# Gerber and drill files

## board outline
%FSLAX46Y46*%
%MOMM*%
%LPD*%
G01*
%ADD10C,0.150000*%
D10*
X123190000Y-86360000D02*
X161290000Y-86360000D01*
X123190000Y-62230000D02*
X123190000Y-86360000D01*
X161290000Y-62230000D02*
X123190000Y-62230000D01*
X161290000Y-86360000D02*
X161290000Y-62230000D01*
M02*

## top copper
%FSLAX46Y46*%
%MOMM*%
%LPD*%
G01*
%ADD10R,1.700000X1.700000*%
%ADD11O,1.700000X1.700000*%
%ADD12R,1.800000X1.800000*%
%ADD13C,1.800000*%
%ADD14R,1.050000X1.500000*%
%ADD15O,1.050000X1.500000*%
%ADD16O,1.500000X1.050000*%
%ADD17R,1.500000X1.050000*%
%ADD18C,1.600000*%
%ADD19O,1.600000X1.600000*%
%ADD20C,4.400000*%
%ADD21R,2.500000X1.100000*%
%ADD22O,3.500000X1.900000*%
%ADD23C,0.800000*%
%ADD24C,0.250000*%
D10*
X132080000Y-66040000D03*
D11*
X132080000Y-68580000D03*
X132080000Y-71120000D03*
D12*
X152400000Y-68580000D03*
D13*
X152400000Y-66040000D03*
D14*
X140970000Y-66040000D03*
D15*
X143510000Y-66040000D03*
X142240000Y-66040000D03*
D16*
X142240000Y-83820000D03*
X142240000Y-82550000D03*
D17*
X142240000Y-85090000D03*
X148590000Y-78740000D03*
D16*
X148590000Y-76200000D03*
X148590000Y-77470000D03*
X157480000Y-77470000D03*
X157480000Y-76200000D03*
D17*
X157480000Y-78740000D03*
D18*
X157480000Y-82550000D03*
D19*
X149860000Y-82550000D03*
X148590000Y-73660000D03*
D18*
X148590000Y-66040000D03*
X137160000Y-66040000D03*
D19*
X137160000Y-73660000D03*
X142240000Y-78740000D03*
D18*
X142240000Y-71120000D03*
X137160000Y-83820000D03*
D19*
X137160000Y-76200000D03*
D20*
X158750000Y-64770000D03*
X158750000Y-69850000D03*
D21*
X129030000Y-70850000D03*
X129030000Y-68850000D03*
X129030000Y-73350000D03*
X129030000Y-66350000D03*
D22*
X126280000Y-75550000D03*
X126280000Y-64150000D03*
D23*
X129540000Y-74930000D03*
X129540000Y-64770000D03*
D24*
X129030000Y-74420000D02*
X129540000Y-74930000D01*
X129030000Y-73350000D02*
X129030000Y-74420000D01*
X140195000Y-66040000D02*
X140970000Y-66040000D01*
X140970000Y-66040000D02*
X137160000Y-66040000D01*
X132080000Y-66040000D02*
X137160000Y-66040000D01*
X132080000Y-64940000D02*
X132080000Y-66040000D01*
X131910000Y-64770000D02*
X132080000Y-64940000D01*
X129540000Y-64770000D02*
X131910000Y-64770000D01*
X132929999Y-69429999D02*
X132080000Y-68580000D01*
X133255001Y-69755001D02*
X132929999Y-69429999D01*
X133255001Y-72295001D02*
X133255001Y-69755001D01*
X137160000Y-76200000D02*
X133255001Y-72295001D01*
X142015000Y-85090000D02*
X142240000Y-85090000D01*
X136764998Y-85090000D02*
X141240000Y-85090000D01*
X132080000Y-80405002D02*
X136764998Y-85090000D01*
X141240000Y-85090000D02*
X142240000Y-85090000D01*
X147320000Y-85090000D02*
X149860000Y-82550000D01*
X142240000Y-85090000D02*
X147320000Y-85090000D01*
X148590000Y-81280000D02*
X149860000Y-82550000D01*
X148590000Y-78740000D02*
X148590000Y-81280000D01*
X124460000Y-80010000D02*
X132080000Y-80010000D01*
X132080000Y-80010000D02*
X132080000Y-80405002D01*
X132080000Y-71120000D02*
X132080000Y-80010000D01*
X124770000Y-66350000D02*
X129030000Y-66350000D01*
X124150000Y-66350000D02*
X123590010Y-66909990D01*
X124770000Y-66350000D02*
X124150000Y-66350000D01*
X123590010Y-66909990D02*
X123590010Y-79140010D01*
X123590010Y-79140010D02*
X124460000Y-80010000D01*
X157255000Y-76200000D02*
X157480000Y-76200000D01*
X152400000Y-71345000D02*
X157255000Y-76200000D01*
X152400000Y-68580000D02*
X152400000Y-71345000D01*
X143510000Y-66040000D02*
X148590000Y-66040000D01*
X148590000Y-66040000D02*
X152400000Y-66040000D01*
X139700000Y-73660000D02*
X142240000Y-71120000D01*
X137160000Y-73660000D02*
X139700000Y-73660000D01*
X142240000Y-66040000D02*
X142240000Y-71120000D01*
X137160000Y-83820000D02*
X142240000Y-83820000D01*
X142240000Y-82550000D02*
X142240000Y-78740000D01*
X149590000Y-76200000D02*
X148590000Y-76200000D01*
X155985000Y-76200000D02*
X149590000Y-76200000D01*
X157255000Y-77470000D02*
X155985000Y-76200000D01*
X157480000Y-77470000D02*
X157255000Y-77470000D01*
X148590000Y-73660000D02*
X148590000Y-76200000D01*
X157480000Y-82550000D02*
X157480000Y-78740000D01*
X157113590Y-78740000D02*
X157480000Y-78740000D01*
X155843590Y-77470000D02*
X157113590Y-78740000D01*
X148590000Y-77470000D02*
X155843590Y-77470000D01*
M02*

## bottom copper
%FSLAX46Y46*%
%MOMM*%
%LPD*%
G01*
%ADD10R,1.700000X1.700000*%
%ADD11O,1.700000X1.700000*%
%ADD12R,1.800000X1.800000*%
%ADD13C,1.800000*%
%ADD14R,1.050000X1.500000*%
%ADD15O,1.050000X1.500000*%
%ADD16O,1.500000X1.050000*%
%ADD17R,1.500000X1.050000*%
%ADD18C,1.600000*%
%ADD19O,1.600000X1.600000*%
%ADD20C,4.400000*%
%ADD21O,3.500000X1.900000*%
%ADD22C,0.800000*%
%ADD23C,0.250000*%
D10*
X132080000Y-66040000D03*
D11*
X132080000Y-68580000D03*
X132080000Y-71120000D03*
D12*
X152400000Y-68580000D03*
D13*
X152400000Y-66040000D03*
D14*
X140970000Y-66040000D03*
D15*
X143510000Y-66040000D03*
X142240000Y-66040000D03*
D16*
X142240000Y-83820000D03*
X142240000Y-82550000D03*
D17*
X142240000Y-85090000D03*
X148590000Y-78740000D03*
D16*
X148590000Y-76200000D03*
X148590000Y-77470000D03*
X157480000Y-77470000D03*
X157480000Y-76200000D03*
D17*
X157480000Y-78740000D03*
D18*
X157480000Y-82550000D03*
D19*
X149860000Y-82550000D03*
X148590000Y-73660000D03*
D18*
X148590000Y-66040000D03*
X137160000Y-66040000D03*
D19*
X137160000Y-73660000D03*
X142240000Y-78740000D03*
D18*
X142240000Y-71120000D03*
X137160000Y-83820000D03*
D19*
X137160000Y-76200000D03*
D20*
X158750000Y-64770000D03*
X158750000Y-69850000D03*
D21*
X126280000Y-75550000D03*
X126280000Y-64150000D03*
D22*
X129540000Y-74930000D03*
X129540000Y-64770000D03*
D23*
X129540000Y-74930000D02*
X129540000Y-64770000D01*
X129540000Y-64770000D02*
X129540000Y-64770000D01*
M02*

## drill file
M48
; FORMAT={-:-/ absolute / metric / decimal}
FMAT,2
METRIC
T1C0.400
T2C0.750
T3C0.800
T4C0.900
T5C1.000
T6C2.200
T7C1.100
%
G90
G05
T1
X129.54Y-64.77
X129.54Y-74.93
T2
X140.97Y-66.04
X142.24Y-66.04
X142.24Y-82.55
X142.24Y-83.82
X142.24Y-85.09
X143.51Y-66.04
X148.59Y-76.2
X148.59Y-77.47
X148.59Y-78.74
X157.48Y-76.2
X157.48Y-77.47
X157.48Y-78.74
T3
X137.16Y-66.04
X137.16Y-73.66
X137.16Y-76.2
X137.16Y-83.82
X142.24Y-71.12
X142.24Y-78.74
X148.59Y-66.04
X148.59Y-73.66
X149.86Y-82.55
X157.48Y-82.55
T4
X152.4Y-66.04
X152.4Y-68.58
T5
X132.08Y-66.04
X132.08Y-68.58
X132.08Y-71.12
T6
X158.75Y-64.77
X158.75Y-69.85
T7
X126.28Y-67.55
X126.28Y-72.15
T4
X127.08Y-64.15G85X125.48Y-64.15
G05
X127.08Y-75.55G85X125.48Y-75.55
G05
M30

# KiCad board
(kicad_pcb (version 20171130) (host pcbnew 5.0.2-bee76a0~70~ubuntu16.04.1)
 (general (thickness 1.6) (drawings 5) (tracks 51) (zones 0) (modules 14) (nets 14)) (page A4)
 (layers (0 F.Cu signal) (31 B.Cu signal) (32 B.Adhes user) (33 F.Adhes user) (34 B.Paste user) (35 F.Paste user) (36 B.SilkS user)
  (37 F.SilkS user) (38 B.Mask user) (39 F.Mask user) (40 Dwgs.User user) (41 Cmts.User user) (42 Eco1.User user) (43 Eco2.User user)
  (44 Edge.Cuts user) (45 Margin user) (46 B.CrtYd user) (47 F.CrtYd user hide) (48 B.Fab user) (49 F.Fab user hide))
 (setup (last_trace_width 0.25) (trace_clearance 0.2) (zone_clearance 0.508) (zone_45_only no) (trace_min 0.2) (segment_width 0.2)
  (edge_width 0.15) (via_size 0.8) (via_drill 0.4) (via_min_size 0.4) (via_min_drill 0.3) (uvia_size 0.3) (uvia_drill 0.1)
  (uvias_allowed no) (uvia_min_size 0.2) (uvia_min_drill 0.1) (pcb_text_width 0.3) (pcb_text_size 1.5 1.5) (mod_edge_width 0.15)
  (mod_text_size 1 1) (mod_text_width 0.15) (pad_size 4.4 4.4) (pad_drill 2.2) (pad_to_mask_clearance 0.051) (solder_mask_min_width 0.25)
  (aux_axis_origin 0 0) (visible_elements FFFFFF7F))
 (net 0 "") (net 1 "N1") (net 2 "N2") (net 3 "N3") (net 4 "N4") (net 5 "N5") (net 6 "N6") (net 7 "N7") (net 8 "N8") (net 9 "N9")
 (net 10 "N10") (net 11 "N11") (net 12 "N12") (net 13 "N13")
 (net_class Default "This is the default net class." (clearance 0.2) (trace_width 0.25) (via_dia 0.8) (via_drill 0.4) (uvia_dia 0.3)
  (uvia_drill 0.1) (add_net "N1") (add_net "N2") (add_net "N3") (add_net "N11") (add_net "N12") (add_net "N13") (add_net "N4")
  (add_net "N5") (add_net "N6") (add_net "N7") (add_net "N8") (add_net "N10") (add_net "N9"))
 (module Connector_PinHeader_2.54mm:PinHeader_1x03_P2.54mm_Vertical (layer F.Cu) (at 132.08 66.04)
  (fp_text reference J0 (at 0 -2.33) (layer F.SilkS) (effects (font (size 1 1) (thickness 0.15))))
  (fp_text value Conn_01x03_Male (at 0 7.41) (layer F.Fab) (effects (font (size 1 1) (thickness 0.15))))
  (pad 1 thru_hole rect (at 0 0) (size 1.7 1.7) (drill 1) (layers *.Cu *.Mask) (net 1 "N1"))
  (pad 2 thru_hole oval (at 0 2.54) (size 1.7 1.7) (drill 1) (layers *.Cu *.Mask) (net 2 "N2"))
  (pad 3 thru_hole oval (at 0 5.08) (size 1.7 1.7) (drill 1) (layers *.Cu *.Mask) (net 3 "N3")))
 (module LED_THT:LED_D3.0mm (layer F.Cu) (at 152.4 68.58 90)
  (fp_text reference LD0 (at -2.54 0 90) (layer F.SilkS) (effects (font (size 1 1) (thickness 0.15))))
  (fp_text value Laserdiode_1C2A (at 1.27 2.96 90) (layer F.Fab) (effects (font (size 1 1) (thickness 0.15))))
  (pad 1 thru_hole rect (at 0 0 90) (size 1.8 1.8) (drill 0.9) (layers *.Cu *.Mask) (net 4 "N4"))
  (pad 2 thru_hole circle (at 2.54 0 90) (size 1.8 1.8) (drill 0.9) (layers *.Cu *.Mask) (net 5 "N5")))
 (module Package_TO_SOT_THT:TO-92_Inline (layer F.Cu) (at 140.97 66.04)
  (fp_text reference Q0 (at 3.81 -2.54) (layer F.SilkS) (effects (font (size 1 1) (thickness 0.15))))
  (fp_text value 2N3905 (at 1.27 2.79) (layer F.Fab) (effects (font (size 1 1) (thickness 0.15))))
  (pad 1 thru_hole rect (at 0 0) (size 1.05 1.5) (drill 0.75) (layers *.Cu *.Mask) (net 1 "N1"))
  (pad 3 thru_hole oval (at 2.54 0) (size 1.05 1.5) (drill 0.75) (layers *.Cu *.Mask) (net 5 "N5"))
  (pad 2 thru_hole oval (at 1.27 0) (size 1.05 1.5) (drill 0.75) (layers *.Cu *.Mask) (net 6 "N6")))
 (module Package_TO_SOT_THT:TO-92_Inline (layer F.Cu) (at 142.24 85.09 90)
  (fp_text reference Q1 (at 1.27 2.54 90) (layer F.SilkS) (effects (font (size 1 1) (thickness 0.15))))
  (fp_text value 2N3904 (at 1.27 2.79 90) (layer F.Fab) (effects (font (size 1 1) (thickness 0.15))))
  (pad 2 thru_hole oval (at 1.27 0 90) (size 1.05 1.5) (drill 0.75) (layers *.Cu *.Mask) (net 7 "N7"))
  (pad 3 thru_hole oval (at 2.54 0 90) (size 1.05 1.5) (drill 0.75) (layers *.Cu *.Mask) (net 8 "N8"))
  (pad 1 thru_hole rect (at 0 0 90) (size 1.05 1.5) (drill 0.75) (layers *.Cu *.Mask) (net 3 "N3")))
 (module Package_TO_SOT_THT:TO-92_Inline (layer F.Cu) (at 148.59 78.74 90)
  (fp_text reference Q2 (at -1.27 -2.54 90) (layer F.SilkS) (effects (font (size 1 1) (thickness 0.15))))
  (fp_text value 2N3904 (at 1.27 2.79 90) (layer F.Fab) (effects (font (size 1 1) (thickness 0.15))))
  (pad 1 thru_hole rect (at 0 0 90) (size 1.05 1.5) (drill 0.75) (layers *.Cu *.Mask) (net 3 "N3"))
  (pad 3 thru_hole oval (at 2.54 0 90) (size 1.05 1.5) (drill 0.75) (layers *.Cu *.Mask) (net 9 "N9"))
  (pad 2 thru_hole oval (at 1.27 0 90) (size 1.05 1.5) (drill 0.75) (layers *.Cu *.Mask) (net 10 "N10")))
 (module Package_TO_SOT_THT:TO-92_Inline (layer F.Cu) (at 157.48 78.74 90)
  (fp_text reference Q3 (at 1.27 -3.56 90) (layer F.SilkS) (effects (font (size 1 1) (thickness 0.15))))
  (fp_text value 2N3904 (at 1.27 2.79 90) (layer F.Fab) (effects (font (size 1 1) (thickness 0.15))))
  (pad 2 thru_hole oval (at 1.27 0 90) (size 1.05 1.5) (drill 0.75) (layers *.Cu *.Mask) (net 9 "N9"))
  (pad 3 thru_hole oval (at 2.54 0 90) (size 1.05 1.5) (drill 0.75) (layers *.Cu *.Mask) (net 4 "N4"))
  (pad 1 thru_hole rect (at 0 0 90) (size 1.05 1.5) (drill 0.75) (layers *.Cu *.Mask) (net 10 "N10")))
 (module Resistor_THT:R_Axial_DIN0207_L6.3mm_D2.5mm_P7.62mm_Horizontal (layer F.Cu) (at 157.48 82.55 180)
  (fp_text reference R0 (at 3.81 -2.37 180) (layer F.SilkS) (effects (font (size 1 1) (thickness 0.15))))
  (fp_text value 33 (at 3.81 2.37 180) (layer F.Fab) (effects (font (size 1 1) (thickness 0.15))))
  (pad 1 thru_hole circle (at 0 0 180) (size 1.6 1.6) (drill 0.8) (layers *.Cu *.Mask) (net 10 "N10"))
  (pad 2 thru_hole oval (at 7.62 0 180) (size 1.6 1.6) (drill 0.8) (layers *.Cu *.Mask) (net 3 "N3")))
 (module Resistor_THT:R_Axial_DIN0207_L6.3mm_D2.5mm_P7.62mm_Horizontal (layer F.Cu) (at 148.59 66.04 270)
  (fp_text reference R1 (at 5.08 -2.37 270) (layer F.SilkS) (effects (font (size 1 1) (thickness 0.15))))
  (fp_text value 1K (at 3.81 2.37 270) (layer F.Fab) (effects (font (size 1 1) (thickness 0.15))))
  (pad 2 thru_hole oval (at 7.62 0 270) (size 1.6 1.6) (drill 0.8) (layers *.Cu *.Mask) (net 9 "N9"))
  (pad 1 thru_hole circle (at 0 0 270) (size 1.6 1.6) (drill 0.8) (layers *.Cu *.Mask) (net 5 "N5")))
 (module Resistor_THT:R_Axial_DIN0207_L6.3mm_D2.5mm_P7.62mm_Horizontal (layer F.Cu) (at 137.16 66.04 270)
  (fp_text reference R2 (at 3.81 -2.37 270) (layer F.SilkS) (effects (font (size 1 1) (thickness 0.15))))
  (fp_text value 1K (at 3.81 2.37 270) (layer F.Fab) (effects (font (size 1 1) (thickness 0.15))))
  (pad 1 thru_hole circle (at 0 0 270) (size 1.6 1.6) (drill 0.8) (layers *.Cu *.Mask) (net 1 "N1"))
  (pad 2 thru_hole oval (at 7.62 0 270) (size 1.6 1.6) (drill 0.8) (layers *.Cu *.Mask) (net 6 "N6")))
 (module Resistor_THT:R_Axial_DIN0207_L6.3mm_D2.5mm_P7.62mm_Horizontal (layer F.Cu) (at 142.24 71.12 270)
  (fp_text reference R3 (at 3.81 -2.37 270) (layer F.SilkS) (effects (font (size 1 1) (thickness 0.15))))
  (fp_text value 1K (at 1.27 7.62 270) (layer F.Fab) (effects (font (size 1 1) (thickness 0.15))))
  (pad 2 thru_hole oval (at 7.62 0 270) (size 1.6 1.6) (drill 0.8) (layers *.Cu *.Mask) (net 8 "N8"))
  (pad 1 thru_hole circle (at 0 0 270) (size 1.6 1.6) (drill 0.8) (layers *.Cu *.Mask) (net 6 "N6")))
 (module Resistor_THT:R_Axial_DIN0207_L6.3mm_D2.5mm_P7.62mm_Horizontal (layer F.Cu) (at 137.16 83.82 90)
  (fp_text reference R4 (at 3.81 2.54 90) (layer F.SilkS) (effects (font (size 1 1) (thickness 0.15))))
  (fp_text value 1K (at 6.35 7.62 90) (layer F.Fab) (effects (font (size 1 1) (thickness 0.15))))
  (pad 1 thru_hole circle (at 0 0 90) (size 1.6 1.6) (drill 0.8) (layers *.Cu *.Mask) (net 7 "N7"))
  (pad 2 thru_hole oval (at 7.62 0 90) (size 1.6 1.6) (drill 0.8) (layers *.Cu *.Mask) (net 2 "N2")))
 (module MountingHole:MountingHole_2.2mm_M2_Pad (layer F.Cu) (at 158.75 64.77)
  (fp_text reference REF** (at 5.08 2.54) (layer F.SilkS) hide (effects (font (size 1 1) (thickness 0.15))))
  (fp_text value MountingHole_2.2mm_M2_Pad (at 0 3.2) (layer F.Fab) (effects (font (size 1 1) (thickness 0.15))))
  (pad "" thru_hole circle (at 0 0) (size 4.4 4.4) (drill 2.2) (layers *.Cu *.Mask)))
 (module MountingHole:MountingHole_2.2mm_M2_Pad (layer F.Cu) (at 158.75 69.85)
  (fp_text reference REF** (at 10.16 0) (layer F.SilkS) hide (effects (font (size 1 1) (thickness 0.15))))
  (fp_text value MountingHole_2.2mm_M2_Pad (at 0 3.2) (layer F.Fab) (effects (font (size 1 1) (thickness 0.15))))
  (pad "" thru_hole circle (at 0 0) (size 4.4 4.4) (drill 2.2) (layers *.Cu *.Mask)))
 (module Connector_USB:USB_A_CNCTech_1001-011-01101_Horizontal (layer F.Cu) (at 119.38 69.85 180)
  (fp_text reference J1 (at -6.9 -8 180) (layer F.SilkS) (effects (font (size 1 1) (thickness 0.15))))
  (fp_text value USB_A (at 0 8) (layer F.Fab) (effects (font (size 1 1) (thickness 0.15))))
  (pad 2 smd rect (at -9.65 -1 180) (size 2.5 1.1) (layers F.Cu F.Paste F.Mask) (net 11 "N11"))
  (pad 3 smd rect (at -9.65 1 180) (size 2.5 1.1) (layers F.Cu F.Paste F.Mask) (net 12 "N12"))
  (pad 1 smd rect (at -9.65 -3.5 180) (size 2.5 1.1) (layers F.Cu F.Paste F.Mask) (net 1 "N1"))
  (pad 4 smd rect (at -9.65 3.5 180) (size 2.5 1.1) (layers F.Cu F.Paste F.Mask) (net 3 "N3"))
  (pad 5 thru_hole oval (at -6.9 -5.7 180) (size 3.5 1.9) (drill oval 2.5 0.9) (layers *.Cu *.Mask) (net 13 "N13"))
  (pad 5 thru_hole oval (at -6.9 5.7 180) (size 3.5 1.9) (drill oval 2.5 0.9) (layers *.Cu *.Mask) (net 13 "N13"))
  (pad "" np_thru_hole circle (at -6.9 -2.3 180) (size 1.1 1.1) (drill 1.1) (layers *.Cu *.Mask))
  (pad "" np_thru_hole circle (at -6.9 2.3 180) (size 1.1 1.1) (drill 1.1) (layers *.Cu *.Mask)))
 (gr_line (start 123.19 86.36) (end 161.29 86.36) (layer Edge.Cuts) (width 0.15))
 (gr_line (start 123.19 62.23) (end 123.19 86.36) (layer Edge.Cuts) (width 0.15))
 (gr_line (start 161.29 62.23) (end 123.19 62.23) (layer Edge.Cuts) (width 0.15))
 (gr_line (start 161.29 86.36) (end 161.29 62.23) (layer Edge.Cuts) (width 0.15))
 (via (at 129.54 74.93) (size 0.8) (drill 0.4) (layers F.Cu B.Cu) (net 1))
 (segment (start 129.03 74.42) (end 129.54 74.93) (width 0.25) (layer F.Cu) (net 1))
 (segment (start 129.03 73.35) (end 129.03 74.42) (width 0.25) (layer F.Cu) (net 1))
 (segment (start 129.54 74.93) (end 129.54 64.77) (width 0.25) (layer B.Cu) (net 1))
 (segment (start 129.54 64.77) (end 129.54 64.77) (width 0.25) (layer B.Cu) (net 1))
 (via (at 129.54 64.77) (size 0.8) (drill 0.4) (layers F.Cu B.Cu) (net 1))
 (segment (start 140.195 66.04) (end 140.97 66.04) (width 0.25) (layer F.Cu) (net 1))
 (segment (start 140.97 66.04) (end 137.16 66.04) (width 0.25) (layer F.Cu) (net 1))
 (segment (start 132.08 66.04) (end 137.16 66.04) (width 0.25) (layer F.Cu) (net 1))
 (segment (start 132.08 64.94) (end 132.08 66.04) (width 0.25) (layer F.Cu) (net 1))
 (segment (start 131.91 64.77) (end 132.08 64.94) (width 0.25) (layer F.Cu) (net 1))
 (segment (start 129.54 64.77) (end 131.91 64.77) (width 0.25) (layer F.Cu) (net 1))
 (segment (start 132.929999 69.429999) (end 132.08 68.58) (width 0.25) (layer F.Cu) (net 2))
 (segment (start 133.255001 69.755001) (end 132.929999 69.429999) (width 0.25) (layer F.Cu) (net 2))
 (segment (start 133.255001 72.295001) (end 133.255001 69.755001) (width 0.25) (layer F.Cu) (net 2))
 (segment (start 137.16 76.2) (end 133.255001 72.295001) (width 0.25) (layer F.Cu) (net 2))
 (segment (start 142.015 85.09) (end 142.24 85.09) (width 0.25) (layer F.Cu) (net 3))
 (segment (start 136.764998 85.09) (end 141.24 85.09) (width 0.25) (layer F.Cu) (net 3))
 (segment (start 132.08 80.405002) (end 136.764998 85.09) (width 0.25) (layer F.Cu) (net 3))
 (segment (start 141.24 85.09) (end 142.24 85.09) (width 0.25) (layer F.Cu) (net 3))
 (segment (start 147.32 85.09) (end 149.86 82.55) (width 0.25) (layer F.Cu) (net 3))
 (segment (start 142.24 85.09) (end 147.32 85.09) (width 0.25) (layer F.Cu) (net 3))
 (segment (start 148.59 81.28) (end 149.86 82.55) (width 0.25) (layer F.Cu) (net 3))
 (segment (start 148.59 78.74) (end 148.59 81.28) (width 0.25) (layer F.Cu) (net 3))
 (segment (start 124.46 80.01) (end 132.08 80.01) (width 0.25) (layer F.Cu) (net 3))
 (segment (start 132.08 80.01) (end 132.08 80.405002) (width 0.25) (layer F.Cu) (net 3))
 (segment (start 132.08 71.12) (end 132.08 80.01) (width 0.25) (layer F.Cu) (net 3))
 (segment (start 124.77 66.35) (end 129.03 66.35) (width 0.25) (layer F.Cu) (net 3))
 (segment (start 124.15 66.35) (end 123.59001 66.90999) (width 0.25) (layer F.Cu) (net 3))
 (segment (start 124.77 66.35) (end 124.15 66.35) (width 0.25) (layer F.Cu) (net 3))
 (segment (start 123.59001 66.90999) (end 123.59001 79.14001) (width 0.25) (layer F.Cu) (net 3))
 (segment (start 123.59001 79.14001) (end 124.46 80.01) (width 0.25) (layer F.Cu) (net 3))
 (segment (start 157.255 76.2) (end 157.48 76.2) (width 0.25) (layer F.Cu) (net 4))
 (segment (start 152.4 71.345) (end 157.255 76.2) (width 0.25) (layer F.Cu) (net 4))
 (segment (start 152.4 68.58) (end 152.4 71.345) (width 0.25) (layer F.Cu) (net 4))
 (segment (start 143.51 66.04) (end 148.59 66.04) (width 0.25) (layer F.Cu) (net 5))
 (segment (start 148.59 66.04) (end 152.4 66.04) (width 0.25) (layer F.Cu) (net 5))
 (segment (start 139.7 73.66) (end 142.24 71.12) (width 0.25) (layer F.Cu) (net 6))
 (segment (start 137.16 73.66) (end 139.7 73.66) (width 0.25) (layer F.Cu) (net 6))
 (segment (start 142.24 66.04) (end 142.24 71.12) (width 0.25) (layer F.Cu) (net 6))
 (segment (start 137.16 83.82) (end 142.24 83.82) (width 0.25) (layer F.Cu) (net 7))
 (segment (start 142.24 82.55) (end 142.24 78.74) (width 0.25) (layer F.Cu) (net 8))
 (segment (start 149.59 76.2) (end 148.59 76.2) (width 0.25) (layer F.Cu) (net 9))
 (segment (start 155.985 76.2) (end 149.59 76.2) (width 0.25) (layer F.Cu) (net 9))
 (segment (start 157.255 77.47) (end 155.985 76.2) (width 0.25) (layer F.Cu) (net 9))
 (segment (start 157.48 77.47) (end 157.255 77.47) (width 0.25) (layer F.Cu) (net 9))
 (segment (start 148.59 73.66) (end 148.59 76.2) (width 0.25) (layer F.Cu) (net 9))
 (segment (start 157.48 82.55) (end 157.48 78.74) (width 0.25) (layer F.Cu) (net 10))
 (segment (start 157.11359 78.74) (end 157.48 78.74) (width 0.25) (layer F.Cu) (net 10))
 (segment (start 155.84359 77.47) (end 157.11359 78.74) (width 0.25) (layer F.Cu) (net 10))
 (segment (start 148.59 77.47) (end 155.84359 77.47) (width 0.25) (layer F.Cu) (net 10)))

